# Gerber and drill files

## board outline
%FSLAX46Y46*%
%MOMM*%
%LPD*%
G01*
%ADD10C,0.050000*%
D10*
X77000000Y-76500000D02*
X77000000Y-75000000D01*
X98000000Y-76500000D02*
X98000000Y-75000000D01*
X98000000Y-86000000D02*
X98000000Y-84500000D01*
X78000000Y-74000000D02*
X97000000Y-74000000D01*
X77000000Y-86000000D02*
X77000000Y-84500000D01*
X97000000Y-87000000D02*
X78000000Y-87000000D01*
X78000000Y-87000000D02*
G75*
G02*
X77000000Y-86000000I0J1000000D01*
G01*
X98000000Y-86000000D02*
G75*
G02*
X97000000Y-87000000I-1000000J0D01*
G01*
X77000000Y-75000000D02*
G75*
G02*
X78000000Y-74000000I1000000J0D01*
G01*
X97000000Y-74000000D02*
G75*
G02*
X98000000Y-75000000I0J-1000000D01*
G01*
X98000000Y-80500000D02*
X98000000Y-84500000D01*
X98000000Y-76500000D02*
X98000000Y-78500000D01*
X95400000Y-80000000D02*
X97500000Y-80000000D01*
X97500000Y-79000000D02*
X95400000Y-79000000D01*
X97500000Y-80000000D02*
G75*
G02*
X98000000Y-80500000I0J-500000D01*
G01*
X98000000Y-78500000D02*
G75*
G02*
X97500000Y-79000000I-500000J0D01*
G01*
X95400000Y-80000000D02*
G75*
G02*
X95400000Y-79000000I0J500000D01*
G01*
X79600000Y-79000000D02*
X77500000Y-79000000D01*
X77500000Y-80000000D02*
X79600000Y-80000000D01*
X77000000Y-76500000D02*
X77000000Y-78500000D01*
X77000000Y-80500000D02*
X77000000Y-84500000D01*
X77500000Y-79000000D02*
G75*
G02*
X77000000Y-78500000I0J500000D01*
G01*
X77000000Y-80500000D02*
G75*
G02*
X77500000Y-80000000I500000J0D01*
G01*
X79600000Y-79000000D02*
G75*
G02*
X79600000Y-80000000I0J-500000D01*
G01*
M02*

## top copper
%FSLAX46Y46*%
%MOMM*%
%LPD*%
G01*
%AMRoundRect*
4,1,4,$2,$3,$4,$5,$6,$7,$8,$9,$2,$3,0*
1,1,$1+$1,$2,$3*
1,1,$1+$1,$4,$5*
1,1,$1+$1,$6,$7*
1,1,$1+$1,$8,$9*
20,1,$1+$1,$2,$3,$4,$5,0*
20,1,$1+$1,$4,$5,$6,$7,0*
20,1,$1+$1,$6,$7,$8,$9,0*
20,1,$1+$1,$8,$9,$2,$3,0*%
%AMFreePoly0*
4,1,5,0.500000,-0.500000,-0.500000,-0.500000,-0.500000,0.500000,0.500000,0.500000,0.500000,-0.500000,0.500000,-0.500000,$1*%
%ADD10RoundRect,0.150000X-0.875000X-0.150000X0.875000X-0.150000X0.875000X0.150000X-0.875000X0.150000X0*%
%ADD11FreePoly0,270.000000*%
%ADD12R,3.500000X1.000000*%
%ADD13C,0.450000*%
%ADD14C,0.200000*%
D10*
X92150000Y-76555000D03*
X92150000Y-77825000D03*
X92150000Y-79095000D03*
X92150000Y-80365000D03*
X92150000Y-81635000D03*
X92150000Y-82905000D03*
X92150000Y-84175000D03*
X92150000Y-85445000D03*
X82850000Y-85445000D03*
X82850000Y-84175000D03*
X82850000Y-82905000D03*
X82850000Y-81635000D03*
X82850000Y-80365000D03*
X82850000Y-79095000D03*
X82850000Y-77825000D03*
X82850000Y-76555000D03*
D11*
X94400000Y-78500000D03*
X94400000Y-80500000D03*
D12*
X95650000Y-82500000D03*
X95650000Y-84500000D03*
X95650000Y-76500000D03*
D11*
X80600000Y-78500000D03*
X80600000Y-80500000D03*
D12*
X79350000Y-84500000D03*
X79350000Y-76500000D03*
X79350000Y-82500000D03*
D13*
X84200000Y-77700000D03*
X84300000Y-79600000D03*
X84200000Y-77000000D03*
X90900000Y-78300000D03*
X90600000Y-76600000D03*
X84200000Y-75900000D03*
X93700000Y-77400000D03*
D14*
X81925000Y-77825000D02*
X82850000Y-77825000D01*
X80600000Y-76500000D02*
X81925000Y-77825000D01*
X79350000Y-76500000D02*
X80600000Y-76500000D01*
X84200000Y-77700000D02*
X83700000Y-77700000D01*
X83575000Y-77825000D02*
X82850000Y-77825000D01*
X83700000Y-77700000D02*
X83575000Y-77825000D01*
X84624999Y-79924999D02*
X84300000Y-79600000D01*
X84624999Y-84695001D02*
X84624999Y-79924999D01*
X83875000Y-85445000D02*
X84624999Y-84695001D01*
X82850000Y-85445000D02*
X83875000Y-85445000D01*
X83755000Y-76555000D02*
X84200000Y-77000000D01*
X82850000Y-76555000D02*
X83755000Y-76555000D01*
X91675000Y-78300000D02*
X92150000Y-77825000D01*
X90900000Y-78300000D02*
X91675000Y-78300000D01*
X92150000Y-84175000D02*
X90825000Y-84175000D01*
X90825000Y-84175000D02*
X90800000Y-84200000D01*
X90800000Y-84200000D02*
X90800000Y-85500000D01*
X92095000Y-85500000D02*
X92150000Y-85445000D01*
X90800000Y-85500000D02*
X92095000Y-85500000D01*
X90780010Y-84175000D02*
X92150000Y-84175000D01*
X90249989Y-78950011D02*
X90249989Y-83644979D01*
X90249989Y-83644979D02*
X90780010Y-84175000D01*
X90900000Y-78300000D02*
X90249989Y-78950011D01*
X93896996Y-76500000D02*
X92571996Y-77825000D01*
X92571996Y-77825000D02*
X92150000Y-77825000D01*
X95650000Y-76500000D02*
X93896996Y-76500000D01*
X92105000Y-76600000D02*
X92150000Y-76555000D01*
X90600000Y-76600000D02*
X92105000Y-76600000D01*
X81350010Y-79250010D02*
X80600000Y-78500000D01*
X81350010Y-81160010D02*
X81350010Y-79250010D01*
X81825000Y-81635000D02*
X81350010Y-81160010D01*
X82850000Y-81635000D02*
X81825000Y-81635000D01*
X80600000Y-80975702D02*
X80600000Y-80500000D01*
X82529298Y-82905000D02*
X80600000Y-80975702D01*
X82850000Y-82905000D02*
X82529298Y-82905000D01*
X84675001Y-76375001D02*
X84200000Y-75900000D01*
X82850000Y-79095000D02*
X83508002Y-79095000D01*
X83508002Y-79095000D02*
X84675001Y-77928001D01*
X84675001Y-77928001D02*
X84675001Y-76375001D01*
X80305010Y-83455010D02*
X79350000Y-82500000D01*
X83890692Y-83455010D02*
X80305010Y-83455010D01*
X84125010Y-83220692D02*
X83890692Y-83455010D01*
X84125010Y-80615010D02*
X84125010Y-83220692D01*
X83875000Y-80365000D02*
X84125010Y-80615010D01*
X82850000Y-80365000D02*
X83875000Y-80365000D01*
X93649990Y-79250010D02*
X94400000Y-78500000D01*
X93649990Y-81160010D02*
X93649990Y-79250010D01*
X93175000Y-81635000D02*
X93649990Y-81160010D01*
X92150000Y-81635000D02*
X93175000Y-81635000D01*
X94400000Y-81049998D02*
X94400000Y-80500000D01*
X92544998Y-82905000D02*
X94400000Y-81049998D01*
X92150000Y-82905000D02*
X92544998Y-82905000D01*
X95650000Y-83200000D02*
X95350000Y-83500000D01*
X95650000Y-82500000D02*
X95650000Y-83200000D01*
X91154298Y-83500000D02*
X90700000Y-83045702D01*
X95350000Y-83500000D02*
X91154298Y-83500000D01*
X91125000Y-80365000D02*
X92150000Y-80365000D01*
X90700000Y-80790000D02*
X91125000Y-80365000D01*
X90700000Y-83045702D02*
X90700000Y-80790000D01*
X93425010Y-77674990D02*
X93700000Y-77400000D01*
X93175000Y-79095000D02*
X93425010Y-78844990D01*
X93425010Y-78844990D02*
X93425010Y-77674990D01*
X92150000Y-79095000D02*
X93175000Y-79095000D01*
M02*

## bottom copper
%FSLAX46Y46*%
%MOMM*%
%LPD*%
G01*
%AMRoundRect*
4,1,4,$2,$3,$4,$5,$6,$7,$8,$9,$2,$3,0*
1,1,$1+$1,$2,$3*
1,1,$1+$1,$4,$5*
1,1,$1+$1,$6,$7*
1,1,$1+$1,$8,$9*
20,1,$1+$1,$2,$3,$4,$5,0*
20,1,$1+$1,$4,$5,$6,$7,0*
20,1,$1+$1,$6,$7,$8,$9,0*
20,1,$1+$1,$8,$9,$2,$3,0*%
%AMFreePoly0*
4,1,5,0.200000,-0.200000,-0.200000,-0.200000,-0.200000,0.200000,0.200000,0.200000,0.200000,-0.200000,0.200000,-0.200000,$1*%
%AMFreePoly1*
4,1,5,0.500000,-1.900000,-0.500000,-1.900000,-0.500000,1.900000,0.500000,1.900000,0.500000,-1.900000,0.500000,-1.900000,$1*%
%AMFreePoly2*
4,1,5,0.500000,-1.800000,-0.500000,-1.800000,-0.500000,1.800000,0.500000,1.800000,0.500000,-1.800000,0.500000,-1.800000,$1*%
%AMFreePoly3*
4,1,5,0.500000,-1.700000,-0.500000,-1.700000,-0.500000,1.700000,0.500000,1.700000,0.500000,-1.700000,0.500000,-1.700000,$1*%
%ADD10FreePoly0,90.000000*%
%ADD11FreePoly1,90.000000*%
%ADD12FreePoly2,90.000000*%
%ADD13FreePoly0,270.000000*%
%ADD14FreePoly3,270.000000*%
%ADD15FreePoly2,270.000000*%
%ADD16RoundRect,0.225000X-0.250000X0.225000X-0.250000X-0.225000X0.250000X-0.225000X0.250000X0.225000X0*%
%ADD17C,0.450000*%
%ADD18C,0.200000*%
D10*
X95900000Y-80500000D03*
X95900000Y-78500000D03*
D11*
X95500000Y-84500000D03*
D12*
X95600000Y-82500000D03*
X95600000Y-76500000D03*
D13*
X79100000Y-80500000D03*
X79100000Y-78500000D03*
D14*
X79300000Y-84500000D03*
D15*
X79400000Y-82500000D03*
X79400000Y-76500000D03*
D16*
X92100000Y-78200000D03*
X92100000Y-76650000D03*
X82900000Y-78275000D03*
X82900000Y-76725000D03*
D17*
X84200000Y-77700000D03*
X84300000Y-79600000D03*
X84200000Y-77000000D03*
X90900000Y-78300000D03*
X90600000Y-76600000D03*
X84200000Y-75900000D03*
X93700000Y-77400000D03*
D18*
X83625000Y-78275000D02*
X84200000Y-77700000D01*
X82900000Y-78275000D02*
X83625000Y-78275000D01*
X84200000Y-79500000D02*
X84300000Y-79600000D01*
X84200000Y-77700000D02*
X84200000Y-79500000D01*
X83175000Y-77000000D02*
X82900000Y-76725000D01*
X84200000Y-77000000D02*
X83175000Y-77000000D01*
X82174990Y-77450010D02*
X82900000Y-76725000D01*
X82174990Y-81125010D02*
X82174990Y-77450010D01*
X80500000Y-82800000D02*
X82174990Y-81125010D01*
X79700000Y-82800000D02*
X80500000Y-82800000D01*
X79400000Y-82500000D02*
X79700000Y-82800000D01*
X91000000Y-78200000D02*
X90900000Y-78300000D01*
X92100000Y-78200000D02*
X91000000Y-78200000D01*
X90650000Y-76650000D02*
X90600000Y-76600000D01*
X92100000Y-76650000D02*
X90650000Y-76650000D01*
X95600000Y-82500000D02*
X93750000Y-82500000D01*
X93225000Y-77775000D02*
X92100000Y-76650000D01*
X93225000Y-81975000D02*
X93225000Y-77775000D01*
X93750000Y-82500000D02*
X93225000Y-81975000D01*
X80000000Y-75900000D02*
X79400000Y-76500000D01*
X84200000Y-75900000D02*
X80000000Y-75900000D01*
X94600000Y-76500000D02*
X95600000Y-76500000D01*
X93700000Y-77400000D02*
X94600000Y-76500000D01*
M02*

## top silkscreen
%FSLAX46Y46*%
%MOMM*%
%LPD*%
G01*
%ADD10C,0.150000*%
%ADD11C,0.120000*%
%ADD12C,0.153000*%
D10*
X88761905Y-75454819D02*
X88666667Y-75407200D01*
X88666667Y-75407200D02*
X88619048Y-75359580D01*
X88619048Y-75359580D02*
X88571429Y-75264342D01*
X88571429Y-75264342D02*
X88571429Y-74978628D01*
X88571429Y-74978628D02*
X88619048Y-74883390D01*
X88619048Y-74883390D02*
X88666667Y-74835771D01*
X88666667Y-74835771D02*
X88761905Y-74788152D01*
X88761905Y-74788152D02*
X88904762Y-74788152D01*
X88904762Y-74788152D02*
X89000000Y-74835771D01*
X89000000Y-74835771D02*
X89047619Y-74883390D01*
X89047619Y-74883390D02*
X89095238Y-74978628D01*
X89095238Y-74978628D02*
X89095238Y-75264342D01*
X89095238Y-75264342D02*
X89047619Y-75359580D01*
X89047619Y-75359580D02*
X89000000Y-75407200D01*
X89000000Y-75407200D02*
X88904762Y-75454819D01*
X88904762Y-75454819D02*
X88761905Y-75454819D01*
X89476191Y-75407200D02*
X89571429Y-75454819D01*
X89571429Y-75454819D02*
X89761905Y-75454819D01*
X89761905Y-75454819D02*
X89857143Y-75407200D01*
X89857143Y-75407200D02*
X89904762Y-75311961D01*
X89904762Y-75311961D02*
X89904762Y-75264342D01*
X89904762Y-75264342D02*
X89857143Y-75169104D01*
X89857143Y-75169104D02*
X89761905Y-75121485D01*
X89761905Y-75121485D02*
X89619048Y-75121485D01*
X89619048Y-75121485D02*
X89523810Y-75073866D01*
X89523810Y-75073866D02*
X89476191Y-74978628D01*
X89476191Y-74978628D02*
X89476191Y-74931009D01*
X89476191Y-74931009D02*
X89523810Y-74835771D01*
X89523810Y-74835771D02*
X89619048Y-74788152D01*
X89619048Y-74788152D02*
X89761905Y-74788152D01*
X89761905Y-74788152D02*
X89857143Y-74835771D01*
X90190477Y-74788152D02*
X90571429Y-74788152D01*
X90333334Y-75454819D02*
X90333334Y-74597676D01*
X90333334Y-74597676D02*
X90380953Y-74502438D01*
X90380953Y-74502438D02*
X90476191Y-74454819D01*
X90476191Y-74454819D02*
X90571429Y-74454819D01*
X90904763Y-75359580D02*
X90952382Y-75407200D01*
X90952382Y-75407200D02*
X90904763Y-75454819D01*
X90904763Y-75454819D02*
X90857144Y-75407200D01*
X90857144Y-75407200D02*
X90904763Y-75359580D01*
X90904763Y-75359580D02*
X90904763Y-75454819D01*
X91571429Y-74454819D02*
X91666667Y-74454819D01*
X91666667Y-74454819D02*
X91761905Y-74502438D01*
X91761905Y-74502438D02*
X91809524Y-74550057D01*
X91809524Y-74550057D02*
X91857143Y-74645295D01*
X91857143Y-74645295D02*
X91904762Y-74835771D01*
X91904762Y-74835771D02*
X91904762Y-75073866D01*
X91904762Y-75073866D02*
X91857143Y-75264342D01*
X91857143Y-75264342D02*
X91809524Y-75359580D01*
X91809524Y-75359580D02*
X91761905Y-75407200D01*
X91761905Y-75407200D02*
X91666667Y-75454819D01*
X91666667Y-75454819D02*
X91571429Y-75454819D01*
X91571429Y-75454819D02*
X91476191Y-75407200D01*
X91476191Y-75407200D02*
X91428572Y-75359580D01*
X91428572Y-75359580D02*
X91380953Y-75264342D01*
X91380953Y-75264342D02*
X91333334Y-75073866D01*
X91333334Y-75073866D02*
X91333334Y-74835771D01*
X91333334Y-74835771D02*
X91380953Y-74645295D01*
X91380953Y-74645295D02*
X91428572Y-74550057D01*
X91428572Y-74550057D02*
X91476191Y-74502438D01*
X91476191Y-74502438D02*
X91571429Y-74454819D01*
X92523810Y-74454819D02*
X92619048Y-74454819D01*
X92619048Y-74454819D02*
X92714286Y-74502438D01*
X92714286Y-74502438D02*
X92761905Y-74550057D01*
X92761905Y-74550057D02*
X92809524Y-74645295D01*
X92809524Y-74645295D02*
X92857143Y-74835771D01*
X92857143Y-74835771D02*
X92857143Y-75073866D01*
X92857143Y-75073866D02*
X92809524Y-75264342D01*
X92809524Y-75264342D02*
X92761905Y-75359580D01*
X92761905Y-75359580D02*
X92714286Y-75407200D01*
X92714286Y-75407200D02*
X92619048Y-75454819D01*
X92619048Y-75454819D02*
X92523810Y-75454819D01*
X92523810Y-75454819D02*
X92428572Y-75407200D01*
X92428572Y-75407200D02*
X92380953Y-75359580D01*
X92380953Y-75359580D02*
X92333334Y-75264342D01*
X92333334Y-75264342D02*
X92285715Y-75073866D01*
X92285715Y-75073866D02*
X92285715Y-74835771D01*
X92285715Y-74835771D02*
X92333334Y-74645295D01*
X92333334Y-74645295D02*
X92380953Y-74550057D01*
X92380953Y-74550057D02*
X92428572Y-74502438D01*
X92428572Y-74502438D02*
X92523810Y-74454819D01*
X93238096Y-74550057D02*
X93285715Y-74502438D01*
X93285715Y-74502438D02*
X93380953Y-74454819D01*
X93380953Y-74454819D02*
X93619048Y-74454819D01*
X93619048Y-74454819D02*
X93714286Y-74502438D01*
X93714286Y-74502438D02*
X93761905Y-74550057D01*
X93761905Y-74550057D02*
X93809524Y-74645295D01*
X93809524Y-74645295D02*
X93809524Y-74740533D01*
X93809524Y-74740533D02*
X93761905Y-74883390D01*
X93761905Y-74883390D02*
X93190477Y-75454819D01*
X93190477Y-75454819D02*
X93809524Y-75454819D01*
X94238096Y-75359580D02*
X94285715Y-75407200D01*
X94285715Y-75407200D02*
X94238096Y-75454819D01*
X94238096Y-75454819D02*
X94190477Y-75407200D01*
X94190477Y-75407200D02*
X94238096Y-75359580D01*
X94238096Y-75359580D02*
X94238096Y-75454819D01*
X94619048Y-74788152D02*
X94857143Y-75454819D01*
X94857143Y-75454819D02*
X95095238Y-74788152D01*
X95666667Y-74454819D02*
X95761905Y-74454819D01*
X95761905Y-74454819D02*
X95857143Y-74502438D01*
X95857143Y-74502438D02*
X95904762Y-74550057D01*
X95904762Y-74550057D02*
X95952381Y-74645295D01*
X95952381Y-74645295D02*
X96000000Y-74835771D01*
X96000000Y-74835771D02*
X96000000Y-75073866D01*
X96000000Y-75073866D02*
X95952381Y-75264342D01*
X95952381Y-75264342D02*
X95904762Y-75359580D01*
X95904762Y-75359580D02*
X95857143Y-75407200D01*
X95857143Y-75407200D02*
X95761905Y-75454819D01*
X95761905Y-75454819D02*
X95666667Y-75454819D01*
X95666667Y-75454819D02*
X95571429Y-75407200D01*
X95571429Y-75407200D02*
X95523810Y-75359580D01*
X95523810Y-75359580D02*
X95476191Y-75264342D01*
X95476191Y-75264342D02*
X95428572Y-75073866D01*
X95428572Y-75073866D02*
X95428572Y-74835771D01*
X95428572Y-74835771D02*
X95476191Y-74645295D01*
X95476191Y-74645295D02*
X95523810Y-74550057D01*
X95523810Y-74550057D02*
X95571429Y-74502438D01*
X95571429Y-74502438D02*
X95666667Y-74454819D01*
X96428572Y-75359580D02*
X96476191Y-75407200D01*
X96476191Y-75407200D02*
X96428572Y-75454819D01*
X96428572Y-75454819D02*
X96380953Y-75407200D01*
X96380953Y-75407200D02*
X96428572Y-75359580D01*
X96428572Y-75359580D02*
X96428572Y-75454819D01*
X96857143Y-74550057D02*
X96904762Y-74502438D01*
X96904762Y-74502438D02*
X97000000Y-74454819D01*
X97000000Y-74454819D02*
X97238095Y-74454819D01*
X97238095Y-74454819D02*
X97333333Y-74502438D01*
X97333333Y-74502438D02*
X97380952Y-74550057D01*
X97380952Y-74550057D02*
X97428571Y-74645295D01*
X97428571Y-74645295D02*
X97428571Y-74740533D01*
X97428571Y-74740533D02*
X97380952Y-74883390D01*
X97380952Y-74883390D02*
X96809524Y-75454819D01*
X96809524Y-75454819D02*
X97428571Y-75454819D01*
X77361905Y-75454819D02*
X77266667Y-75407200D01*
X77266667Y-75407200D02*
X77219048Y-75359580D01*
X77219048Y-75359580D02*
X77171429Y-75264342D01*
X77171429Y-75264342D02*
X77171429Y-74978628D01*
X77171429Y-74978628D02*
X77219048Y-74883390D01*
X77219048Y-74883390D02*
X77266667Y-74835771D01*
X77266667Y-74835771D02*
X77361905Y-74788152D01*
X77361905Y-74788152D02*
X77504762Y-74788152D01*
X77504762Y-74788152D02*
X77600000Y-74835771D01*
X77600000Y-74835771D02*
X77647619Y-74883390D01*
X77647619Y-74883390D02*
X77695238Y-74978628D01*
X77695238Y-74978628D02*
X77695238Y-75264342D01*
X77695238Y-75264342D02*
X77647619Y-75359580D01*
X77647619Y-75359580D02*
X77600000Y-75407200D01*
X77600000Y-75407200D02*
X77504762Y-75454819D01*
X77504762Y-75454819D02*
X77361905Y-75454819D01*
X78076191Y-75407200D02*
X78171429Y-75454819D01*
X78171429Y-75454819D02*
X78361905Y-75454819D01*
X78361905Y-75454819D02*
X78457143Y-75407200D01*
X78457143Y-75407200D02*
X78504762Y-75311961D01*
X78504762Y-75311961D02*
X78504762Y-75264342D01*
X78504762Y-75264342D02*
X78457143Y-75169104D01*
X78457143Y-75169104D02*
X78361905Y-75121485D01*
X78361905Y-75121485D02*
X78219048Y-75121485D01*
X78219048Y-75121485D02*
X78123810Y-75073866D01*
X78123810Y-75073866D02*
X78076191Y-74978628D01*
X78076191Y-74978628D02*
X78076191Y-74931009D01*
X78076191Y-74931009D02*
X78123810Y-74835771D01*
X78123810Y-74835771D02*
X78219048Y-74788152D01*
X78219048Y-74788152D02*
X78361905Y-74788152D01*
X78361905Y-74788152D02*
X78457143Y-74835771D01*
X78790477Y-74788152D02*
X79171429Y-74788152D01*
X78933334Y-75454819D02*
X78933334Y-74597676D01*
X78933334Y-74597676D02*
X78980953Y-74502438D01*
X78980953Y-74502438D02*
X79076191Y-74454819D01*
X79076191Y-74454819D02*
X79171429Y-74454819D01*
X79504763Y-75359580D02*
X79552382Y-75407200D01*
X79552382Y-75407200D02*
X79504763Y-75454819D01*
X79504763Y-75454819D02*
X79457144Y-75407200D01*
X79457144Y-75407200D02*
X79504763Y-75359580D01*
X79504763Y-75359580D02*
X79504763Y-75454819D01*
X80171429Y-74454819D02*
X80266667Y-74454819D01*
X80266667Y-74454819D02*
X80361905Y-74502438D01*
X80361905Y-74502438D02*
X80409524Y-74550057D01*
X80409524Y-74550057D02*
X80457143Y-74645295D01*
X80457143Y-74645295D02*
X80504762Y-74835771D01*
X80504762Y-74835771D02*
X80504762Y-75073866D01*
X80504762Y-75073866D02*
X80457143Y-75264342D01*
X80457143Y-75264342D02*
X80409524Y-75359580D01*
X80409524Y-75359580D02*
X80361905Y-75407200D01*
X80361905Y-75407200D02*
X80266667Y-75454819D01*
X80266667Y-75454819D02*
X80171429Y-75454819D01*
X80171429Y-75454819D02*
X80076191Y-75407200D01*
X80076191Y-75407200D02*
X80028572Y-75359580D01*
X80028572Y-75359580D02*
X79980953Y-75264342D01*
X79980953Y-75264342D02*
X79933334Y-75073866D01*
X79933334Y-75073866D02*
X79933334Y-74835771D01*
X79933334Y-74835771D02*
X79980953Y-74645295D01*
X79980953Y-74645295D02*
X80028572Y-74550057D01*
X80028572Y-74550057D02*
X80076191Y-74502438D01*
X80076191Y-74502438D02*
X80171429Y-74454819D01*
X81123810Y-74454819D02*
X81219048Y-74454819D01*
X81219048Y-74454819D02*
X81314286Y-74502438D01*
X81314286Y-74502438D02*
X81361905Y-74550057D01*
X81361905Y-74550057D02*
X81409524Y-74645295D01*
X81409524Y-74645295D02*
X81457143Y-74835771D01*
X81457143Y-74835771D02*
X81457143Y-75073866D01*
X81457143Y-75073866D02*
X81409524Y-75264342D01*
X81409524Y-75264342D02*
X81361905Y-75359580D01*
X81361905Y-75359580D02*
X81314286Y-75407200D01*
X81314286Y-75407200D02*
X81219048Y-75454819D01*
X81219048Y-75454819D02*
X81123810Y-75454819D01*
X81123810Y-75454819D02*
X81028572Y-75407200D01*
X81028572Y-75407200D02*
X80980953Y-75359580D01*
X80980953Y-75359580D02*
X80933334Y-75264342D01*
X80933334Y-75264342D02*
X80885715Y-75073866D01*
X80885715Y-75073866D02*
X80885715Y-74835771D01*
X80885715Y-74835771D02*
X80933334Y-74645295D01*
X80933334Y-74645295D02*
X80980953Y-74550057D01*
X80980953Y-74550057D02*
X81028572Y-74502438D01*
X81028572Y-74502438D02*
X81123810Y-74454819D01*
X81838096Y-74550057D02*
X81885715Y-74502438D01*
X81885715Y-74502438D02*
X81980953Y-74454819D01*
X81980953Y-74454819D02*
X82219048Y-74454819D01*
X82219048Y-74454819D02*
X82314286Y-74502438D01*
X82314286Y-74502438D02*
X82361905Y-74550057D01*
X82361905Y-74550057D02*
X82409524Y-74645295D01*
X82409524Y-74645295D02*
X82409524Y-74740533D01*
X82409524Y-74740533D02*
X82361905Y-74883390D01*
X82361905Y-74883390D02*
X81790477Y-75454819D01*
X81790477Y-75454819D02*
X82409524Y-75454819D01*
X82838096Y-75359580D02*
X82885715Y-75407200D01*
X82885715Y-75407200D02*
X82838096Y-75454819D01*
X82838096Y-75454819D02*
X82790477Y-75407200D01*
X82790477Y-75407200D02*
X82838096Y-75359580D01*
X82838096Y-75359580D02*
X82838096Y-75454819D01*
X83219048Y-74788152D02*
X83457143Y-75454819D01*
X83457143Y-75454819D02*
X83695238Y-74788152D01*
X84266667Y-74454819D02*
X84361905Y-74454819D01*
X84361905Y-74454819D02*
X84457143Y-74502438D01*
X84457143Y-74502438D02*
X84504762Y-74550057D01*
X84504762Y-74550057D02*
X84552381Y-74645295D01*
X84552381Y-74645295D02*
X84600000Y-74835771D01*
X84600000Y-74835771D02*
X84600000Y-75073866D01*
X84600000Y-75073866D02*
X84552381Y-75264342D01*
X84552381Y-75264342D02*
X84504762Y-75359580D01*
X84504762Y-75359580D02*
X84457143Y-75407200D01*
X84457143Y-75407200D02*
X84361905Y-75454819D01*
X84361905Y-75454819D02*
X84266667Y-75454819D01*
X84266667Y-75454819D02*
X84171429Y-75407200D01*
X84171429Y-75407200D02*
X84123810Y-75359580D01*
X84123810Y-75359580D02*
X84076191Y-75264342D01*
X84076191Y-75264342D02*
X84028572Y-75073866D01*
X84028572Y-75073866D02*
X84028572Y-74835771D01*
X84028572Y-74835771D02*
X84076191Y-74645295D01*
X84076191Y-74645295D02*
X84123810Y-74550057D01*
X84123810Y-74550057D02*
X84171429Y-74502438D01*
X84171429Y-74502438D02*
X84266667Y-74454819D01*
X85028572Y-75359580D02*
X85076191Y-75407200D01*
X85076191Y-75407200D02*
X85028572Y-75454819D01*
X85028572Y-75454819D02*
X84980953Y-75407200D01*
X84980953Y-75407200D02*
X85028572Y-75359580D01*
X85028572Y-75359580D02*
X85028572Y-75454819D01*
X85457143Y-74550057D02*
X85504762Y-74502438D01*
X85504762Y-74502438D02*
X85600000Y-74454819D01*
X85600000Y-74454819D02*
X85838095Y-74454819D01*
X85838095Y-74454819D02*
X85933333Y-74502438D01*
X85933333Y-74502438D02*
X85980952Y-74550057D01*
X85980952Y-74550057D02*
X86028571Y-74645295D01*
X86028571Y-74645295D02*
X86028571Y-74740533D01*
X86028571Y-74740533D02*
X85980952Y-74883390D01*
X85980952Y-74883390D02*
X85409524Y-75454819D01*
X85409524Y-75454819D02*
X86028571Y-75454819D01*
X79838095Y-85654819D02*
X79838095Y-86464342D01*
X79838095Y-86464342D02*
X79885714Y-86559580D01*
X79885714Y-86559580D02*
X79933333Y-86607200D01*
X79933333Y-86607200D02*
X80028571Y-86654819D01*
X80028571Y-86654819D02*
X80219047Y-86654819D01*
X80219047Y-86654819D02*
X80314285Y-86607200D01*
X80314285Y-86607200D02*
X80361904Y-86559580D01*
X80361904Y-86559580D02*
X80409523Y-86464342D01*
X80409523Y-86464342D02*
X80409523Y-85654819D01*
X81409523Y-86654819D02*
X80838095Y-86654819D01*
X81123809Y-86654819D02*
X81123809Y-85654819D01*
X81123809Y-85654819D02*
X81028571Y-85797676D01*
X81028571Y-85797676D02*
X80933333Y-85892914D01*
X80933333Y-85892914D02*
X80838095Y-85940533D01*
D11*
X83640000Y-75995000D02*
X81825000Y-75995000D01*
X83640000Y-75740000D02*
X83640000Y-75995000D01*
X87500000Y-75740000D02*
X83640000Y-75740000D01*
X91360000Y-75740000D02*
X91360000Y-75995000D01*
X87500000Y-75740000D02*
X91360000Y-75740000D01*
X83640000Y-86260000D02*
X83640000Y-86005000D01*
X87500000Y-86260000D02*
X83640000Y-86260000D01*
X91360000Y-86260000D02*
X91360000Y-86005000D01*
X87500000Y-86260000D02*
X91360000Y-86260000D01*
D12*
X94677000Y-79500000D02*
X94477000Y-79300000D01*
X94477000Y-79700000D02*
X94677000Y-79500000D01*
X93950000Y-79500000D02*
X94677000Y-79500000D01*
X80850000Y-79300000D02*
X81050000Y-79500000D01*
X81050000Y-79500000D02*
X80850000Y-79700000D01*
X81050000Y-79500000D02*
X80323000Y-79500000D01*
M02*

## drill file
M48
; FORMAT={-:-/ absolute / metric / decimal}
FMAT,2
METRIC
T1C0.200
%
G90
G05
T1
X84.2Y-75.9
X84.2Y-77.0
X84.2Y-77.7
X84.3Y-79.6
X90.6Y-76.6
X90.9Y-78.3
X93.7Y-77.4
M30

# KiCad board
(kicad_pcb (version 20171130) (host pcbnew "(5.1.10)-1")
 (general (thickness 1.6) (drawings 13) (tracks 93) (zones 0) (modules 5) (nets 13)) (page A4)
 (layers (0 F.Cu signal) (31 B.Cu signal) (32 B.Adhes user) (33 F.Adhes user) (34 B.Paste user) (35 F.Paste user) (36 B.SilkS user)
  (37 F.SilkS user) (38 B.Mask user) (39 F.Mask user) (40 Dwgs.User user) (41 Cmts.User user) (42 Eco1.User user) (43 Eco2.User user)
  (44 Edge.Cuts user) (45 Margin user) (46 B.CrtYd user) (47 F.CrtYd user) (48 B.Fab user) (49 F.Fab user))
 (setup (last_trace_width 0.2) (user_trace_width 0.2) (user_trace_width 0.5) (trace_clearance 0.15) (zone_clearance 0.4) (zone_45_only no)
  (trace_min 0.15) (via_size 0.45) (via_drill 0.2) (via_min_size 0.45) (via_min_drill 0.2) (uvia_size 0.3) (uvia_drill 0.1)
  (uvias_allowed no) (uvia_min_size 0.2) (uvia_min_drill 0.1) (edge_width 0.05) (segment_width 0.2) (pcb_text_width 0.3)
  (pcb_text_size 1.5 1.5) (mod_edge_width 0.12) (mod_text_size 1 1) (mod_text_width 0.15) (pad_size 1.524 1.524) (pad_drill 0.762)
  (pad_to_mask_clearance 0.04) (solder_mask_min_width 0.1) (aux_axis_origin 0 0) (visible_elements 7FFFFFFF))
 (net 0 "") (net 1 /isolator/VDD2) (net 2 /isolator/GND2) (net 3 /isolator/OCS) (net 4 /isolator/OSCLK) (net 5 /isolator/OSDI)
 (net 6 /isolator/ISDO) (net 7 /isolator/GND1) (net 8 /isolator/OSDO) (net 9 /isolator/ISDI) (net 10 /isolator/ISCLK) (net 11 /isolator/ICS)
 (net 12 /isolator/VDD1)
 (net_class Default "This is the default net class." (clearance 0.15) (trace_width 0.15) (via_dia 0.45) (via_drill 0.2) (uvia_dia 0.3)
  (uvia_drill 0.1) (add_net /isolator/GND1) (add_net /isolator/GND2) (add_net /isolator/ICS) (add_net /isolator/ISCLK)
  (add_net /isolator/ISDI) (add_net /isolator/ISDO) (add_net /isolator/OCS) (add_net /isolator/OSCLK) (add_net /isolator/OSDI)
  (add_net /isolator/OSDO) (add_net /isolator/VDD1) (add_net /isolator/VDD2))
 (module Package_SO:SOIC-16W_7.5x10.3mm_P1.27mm (layer F.Cu) (at 87.5 81)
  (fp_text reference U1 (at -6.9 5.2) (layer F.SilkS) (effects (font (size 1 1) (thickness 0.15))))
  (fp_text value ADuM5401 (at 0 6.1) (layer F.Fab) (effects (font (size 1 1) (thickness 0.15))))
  (fp_line (start -3.86 -5.005) (end -5.675 -5.005) (layer F.SilkS) (width 0.12))
  (fp_line (start -3.86 -5.26) (end -3.86 -5.005) (layer F.SilkS) (width 0.12))
  (fp_line (start 0 -5.26) (end -3.86 -5.26) (layer F.SilkS) (width 0.12))
  (fp_line (start 3.86 -5.26) (end 3.86 -5.005) (layer F.SilkS) (width 0.12))
  (fp_line (start 0 -5.26) (end 3.86 -5.26) (layer F.SilkS) (width 0.12))
  (fp_line (start -3.86 5.26) (end -3.86 5.005) (layer F.SilkS) (width 0.12))
  (fp_line (start 0 5.26) (end -3.86 5.26) (layer F.SilkS) (width 0.12))
  (fp_line (start 3.86 5.26) (end 3.86 5.005) (layer F.SilkS) (width 0.12))
  (fp_line (start 0 5.26) (end 3.86 5.26) (layer F.SilkS) (width 0.12))
  (pad 16 smd roundrect (at 4.65 -4.445) (size 2.05 0.6) (layers F.Cu F.Paste F.Mask) (roundrect_rratio 0.25) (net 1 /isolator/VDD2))
  (pad 15 smd roundrect (at 4.65 -3.175) (size 2.05 0.6) (layers F.Cu F.Paste F.Mask) (roundrect_rratio 0.25) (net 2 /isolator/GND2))
  (pad 14 smd roundrect (at 4.65 -1.905) (size 2.05 0.6) (layers F.Cu F.Paste F.Mask) (roundrect_rratio 0.25) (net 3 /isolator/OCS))
  (pad 13 smd roundrect (at 4.65 -0.635) (size 2.05 0.6) (layers F.Cu F.Paste F.Mask) (roundrect_rratio 0.25) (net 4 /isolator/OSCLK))
  (pad 12 smd roundrect (at 4.65 0.635) (size 2.05 0.6) (layers F.Cu F.Paste F.Mask) (roundrect_rratio 0.25) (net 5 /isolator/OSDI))
  (pad 11 smd roundrect (at 4.65 1.905) (size 2.05 0.6) (layers F.Cu F.Paste F.Mask) (roundrect_rratio 0.25) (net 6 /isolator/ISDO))
  (pad 10 smd roundrect (at 4.65 3.175) (size 2.05 0.6) (layers F.Cu F.Paste F.Mask) (roundrect_rratio 0.25) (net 2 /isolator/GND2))
  (pad 9 smd roundrect (at 4.65 4.445) (size 2.05 0.6) (layers F.Cu F.Paste F.Mask) (roundrect_rratio 0.25) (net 2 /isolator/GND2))
  (pad 8 smd roundrect (at -4.65 4.445) (size 2.05 0.6) (layers F.Cu F.Paste F.Mask) (roundrect_rratio 0.25) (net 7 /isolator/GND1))
  (pad 7 smd roundrect (at -4.65 3.175) (size 2.05 0.6) (layers F.Cu F.Paste F.Mask) (roundrect_rratio 0.25))
  (pad 6 smd roundrect (at -4.65 1.905) (size 2.05 0.6) (layers F.Cu F.Paste F.Mask) (roundrect_rratio 0.25) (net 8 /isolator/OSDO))
  (pad 5 smd roundrect (at -4.65 0.635) (size 2.05 0.6) (layers F.Cu F.Paste F.Mask) (roundrect_rratio 0.25) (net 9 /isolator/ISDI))
  (pad 4 smd roundrect (at -4.65 -0.635) (size 2.05 0.6) (layers F.Cu F.Paste F.Mask) (roundrect_rratio 0.25) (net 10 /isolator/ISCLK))
  (pad 3 smd roundrect (at -4.65 -1.905) (size 2.05 0.6) (layers F.Cu F.Paste F.Mask) (roundrect_rratio 0.25) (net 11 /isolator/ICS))
  (pad 2 smd roundrect (at -4.65 -3.175) (size 2.05 0.6) (layers F.Cu F.Paste F.Mask) (roundrect_rratio 0.25) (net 7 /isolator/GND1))
  (pad 1 smd roundrect (at -4.65 -4.445) (size 2.05 0.6) (layers F.Cu F.Paste F.Mask) (roundrect_rratio 0.25) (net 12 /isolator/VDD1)))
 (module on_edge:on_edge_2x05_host (layer F.Cu) (at 98 80.5 270)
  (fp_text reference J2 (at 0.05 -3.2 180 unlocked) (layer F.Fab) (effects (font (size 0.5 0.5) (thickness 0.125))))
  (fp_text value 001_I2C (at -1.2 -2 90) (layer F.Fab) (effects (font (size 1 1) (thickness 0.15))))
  (fp_line (start 0 0) (end 4 0) (layer Edge.Cuts) (width 0.05))
  (fp_line (start -4 0) (end -2 0) (layer Edge.Cuts) (width 0.05))
  (fp_line (start -0.5 2.6) (end -0.5 0.5) (layer Edge.Cuts) (width 0.05))
  (fp_line (start -1.5 0.5) (end -1.5 2.6) (layer Edge.Cuts) (width 0.05))
  (fp_line (start -1 3.323) (end -1.2 3.523) (layer F.SilkS) (width 0.153))
  (fp_line (start -0.8 3.523) (end -1 3.323) (layer F.SilkS) (width 0.153))
  (fp_line (start -1 4.05) (end -1 3.323) (layer F.SilkS) (width 0.153))
  (fp_arc (start 0 0.5) (end 0 0) (angle -90) (layer Edge.Cuts) (width 0.05))
  (fp_arc (start -2 0.5) (end -1.5 0.5) (angle -90) (layer Edge.Cuts) (width 0.05))
  (fp_arc (start -1 2.6) (end -1.5 2.6) (angle -180) (layer Edge.Cuts) (width 0.05))
  (pad 2 smd custom (at -2 3.6 270) (size 1 1) (layers F.Cu F.Mask) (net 5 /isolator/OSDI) (zone_connect 0)
   (options (clearance outline) (anchor rect)) (primitives))
  (pad 3 smd custom (at 0 3.6 270) (size 1 1) (layers F.Cu F.Mask) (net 6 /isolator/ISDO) (zone_connect 0)
   (options (clearance outline) (anchor rect)) (primitives))
  (pad 8 smd custom (at 0 2.1 90) (size 0.4 0.4) (layers B.Cu B.Mask) (zone_connect 0) (options (clearance outline) (anchor rect))
   (primitives))
  (pad 7 smd custom (at -2 2.1 90) (size 0.4 0.4) (layers B.Cu B.Mask) (zone_connect 0) (options (clearance outline) (anchor rect))
   (primitives))
  (pad 4 smd rect (at 2 2.35 270) (size 1 3.5) (layers F.Cu F.Mask) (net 4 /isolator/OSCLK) (zone_connect 0))
  (pad 10 smd custom (at 4 2.5 90) (size 1 3.8) (layers B.Cu B.Mask) (zone_connect 0) (options (clearance outline) (anchor rect))
   (primitives))
  (pad 9 smd custom (at 2 2.4 90) (size 1 3.6) (layers B.Cu B.Mask) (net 1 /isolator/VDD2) (zone_connect 0)
   (options (clearance outline) (anchor rect)) (primitives))
  (pad 6 smd custom (at -4 2.4 90) (size 1 3.6) (layers B.Cu B.Mask) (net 3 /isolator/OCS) (zone_connect 0)
   (options (clearance outline) (anchor rect)) (primitives))
  (pad 5 smd rect (at 4 2.35 270) (size 1 3.5) (layers F.Cu F.Mask) (zone_connect 0))
  (pad 1 smd rect (at -4 2.35 270) (size 1 3.5) (layers F.Cu F.Mask) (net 2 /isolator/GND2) (zone_connect 0)))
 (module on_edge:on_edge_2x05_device (layer F.Cu) (at 77 80.5 270)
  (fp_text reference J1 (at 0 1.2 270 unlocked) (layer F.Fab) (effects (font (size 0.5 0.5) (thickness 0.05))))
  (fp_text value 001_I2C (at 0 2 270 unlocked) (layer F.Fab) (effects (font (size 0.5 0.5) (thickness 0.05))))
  (fp_line (start -1.5 -2.6) (end -1.5 -0.5) (layer Edge.Cuts) (width 0.05))
  (fp_line (start -0.5 -0.5) (end -0.5 -2.6) (layer Edge.Cuts) (width 0.05))
  (fp_line (start -1.2 -3.85) (end -1 -4.05) (layer F.SilkS) (width 0.153))
  (fp_line (start -1 -4.05) (end -0.8 -3.85) (layer F.SilkS) (width 0.153))
  (fp_line (start -1 -4.05) (end -1 -3.323) (layer F.SilkS) (width 0.153))
  (fp_line (start -4 0) (end -2 0) (layer Edge.Cuts) (width 0.05))
  (fp_line (start 0 0) (end 4 0) (layer Edge.Cuts) (width 0.05))
  (fp_arc (start -2 -0.5) (end -2 0) (angle -90) (layer Edge.Cuts) (width 0.05))
  (fp_arc (start 0 -0.5) (end -0.5 -0.5) (angle -90) (layer Edge.Cuts) (width 0.05))
  (fp_arc (start -1 -2.6) (end -0.5 -2.6) (angle -180) (layer Edge.Cuts) (width 0.05))
  (pad 2 smd custom (at -2 -3.6 270) (size 1 1) (layers F.Cu F.Mask) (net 9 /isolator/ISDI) (zone_connect 0)
   (options (clearance outline) (anchor rect)) (primitives))
  (pad 3 smd custom (at 0 -3.6 270) (size 1 1) (layers F.Cu F.Mask) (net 8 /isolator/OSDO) (zone_connect 0)
   (options (clearance outline) (anchor rect)) (primitives))
  (pad 8 smd custom (at 0 -2.1 270) (size 0.4 0.4) (layers B.Cu B.Mask) (zone_connect 0) (options (clearance outline) (anchor rect))
   (primitives))
  (pad 7 smd custom (at -2 -2.1 270) (size 0.4 0.4) (layers B.Cu B.Mask) (zone_connect 0) (options (clearance outline) (anchor rect))
   (primitives))
  (pad 10 smd custom (at 4 -2.3 270) (size 1 3.4) (layers B.Cu B.Mask) (zone_connect 0) (options (clearance outline) (anchor rect))
   (primitives))
  (pad 9 smd custom (at 2 -2.4 270) (size 1 3.6) (layers B.Cu B.Mask) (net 12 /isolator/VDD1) (zone_connect 0)
   (options (clearance outline) (anchor rect)) (primitives))
  (pad 6 smd custom (at -4 -2.4 270) (size 1 3.6) (layers B.Cu B.Mask) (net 11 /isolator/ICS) (zone_connect 0)
   (options (clearance outline) (anchor rect)) (primitives))
  (pad 5 smd rect (at 4 -2.35 90) (size 1 3.5) (layers F.Cu F.Mask) (zone_connect 0))
  (pad 1 smd rect (at -4 -2.35 90) (size 1 3.5) (layers F.Cu F.Mask) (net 7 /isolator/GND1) (zone_connect 0))
  (pad 4 smd rect (at 2 -2.35 90) (size 1 3.5) (layers F.Cu F.Mask) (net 10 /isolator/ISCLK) (zone_connect 0)))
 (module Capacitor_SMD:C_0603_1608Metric (layer B.Cu) (at 92.1 77.425 270)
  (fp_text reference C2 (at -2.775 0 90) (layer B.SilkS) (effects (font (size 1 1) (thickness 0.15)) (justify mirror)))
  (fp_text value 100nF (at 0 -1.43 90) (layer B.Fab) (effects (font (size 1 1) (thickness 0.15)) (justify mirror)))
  (pad 2 smd roundrect (at 0.775 0 270) (size 0.9 0.95) (layers B.Cu B.Paste B.Mask) (roundrect_rratio 0.25) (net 2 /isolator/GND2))
  (pad 1 smd roundrect (at -0.775 0 270) (size 0.9 0.95) (layers B.Cu B.Paste B.Mask) (roundrect_rratio 0.25) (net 1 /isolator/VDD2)))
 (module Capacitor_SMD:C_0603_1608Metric (layer B.Cu) (at 82.9 77.5 270)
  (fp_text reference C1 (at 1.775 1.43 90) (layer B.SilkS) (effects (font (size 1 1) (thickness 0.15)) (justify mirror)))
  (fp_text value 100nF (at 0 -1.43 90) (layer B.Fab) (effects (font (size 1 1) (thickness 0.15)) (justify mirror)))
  (pad 2 smd roundrect (at 0.775 0 270) (size 0.9 0.95) (layers B.Cu B.Paste B.Mask) (roundrect_rratio 0.25) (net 7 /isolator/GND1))
  (pad 1 smd roundrect (at -0.775 0 270) (size 0.9 0.95) (layers B.Cu B.Paste B.Mask) (roundrect_rratio 0.25) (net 12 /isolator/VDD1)))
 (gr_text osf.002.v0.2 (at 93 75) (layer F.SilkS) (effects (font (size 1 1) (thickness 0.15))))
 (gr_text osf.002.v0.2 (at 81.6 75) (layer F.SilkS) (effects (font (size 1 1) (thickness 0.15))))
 (gr_line (start 77 76.5) (end 77 75) (layer Edge.Cuts) (width 0.05))
 (gr_line (start 98 76.5) (end 98 75) (layer Edge.Cuts) (width 0.05))
 (gr_line (start 98 86) (end 98 84.5) (layer Edge.Cuts) (width 0.05))
 (gr_line (start 78 74) (end 97 74) (layer Edge.Cuts) (width 0.05))
 (gr_line (start 77 86) (end 77 84.5) (layer Edge.Cuts) (width 0.05))
 (gr_line (start 97 87) (end 78 87) (layer Edge.Cuts) (width 0.05))
 (gr_arc (start 78 86) (end 77 86) (angle -90) (layer Edge.Cuts) (width 0.05))
 (gr_arc (start 97 86) (end 97 87) (angle -90) (layer Edge.Cuts) (width 0.05))
 (gr_arc (start 78 75) (end 78 74) (angle -90) (layer Edge.Cuts) (width 0.05))
 (gr_arc (start 97 75) (end 98 75) (angle -90) (layer Edge.Cuts) (width 0.05))
 (segment (start 81.925 77.825) (end 82.85 77.825) (width 0.2) (layer F.Cu) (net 7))
 (segment (start 80.6 76.5) (end 81.925 77.825) (width 0.2) (layer F.Cu) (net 7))
 (segment (start 79.35 76.5) (end 80.6 76.5) (width 0.2) (layer F.Cu) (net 7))
 (via (at 84.2 77.7) (size 0.45) (drill 0.2) (layers F.Cu B.Cu) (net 7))
 (segment (start 84.2 77.7) (end 83.7 77.7) (width 0.2) (layer F.Cu) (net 7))
 (segment (start 83.575 77.825) (end 82.85 77.825) (width 0.2) (layer F.Cu) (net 7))
 (segment (start 83.7 77.7) (end 83.575 77.825) (width 0.2) (layer F.Cu) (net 7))
 (segment (start 83.625 78.275) (end 84.2 77.7) (width 0.2) (layer B.Cu) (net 7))
 (segment (start 82.9 78.275) (end 83.625 78.275) (width 0.2) (layer B.Cu) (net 7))
 (segment (start 84.624999 79.924999) (end 84.3 79.6) (width 0.2) (layer F.Cu) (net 7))
 (segment (start 84.624999 84.695001) (end 84.624999 79.924999) (width 0.2) (layer F.Cu) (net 7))
 (segment (start 83.875 85.445) (end 84.624999 84.695001) (width 0.2) (layer F.Cu) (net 7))
 (segment (start 82.85 85.445) (end 83.875 85.445) (width 0.2) (layer F.Cu) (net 7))
 (segment (start 84.2 79.5) (end 84.3 79.6) (width 0.2) (layer B.Cu) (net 7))
 (segment (start 84.2 77.7) (end 84.2 79.5) (width 0.2) (layer B.Cu) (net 7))
 (via (at 84.3 79.6) (size 0.45) (drill 0.2) (layers F.Cu B.Cu) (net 7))
 (via (at 84.2 77) (size 0.45) (drill 0.2) (layers F.Cu B.Cu) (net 12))
 (segment (start 83.755 76.555) (end 84.2 77) (width 0.2) (layer F.Cu) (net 12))
 (segment (start 82.85 76.555) (end 83.755 76.555) (width 0.2) (layer F.Cu) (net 12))
 (segment (start 83.175 77) (end 82.9 76.725) (width 0.2) (layer B.Cu) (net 12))
 (segment (start 84.2 77) (end 83.175 77) (width 0.2) (layer B.Cu) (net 12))
 (segment (start 82.17499 77.45001) (end 82.9 76.725) (width 0.2) (layer B.Cu) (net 12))
 (segment (start 82.17499 81.12501) (end 82.17499 77.45001) (width 0.2) (layer B.Cu) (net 12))
 (segment (start 80.5 82.8) (end 82.17499 81.12501) (width 0.2) (layer B.Cu) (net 12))
 (segment (start 79.7 82.8) (end 80.5 82.8) (width 0.2) (layer B.Cu) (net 12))
 (segment (start 79.4 82.5) (end 79.7 82.8) (width 0.2) (layer B.Cu) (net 12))
 (segment (start 91 78.2) (end 90.9 78.3) (width 0.2) (layer B.Cu) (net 2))
 (segment (start 92.1 78.2) (end 91 78.2) (width 0.2) (layer B.Cu) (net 2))
 (via (at 90.9 78.3) (size 0.45) (drill 0.2) (layers F.Cu B.Cu) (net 2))
 (segment (start 91.675 78.3) (end 92.15 77.825) (width 0.2) (layer F.Cu) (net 2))
 (segment (start 90.9 78.3) (end 91.675 78.3) (width 0.2) (layer F.Cu) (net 2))
 (segment (start 92.15 84.175) (end 90.825 84.175) (width 0.2) (layer F.Cu) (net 2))
 (segment (start 90.825 84.175) (end 90.8 84.2) (width 0.2) (layer F.Cu) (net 2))
 (segment (start 90.8 84.2) (end 90.8 85.5) (width 0.2) (layer F.Cu) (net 2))
 (segment (start 92.095 85.5) (end 92.15 85.445) (width 0.2) (layer F.Cu) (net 2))
 (segment (start 90.8 85.5) (end 92.095 85.5) (width 0.2) (layer F.Cu) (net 2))
 (segment (start 90.78001 84.175) (end 92.15 84.175) (width 0.2) (layer F.Cu) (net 2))
 (segment (start 90.249989 78.950011) (end 90.249989 83.644979) (width 0.2) (layer F.Cu) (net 2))
 (segment (start 90.249989 83.644979) (end 90.78001 84.175) (width 0.2) (layer F.Cu) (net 2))
 (segment (start 90.9 78.3) (end 90.249989 78.950011) (width 0.2) (layer F.Cu) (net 2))
 (segment (start 93.896996 76.5) (end 92.571996 77.825) (width 0.2) (layer F.Cu) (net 2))
 (segment (start 92.571996 77.825) (end 92.15 77.825) (width 0.2) (layer F.Cu) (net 2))
 (segment (start 95.65 76.5) (end 93.896996 76.5) (width 0.2) (layer F.Cu) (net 2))
 (segment (start 90.65 76.65) (end 90.6 76.6) (width 0.2) (layer B.Cu) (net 1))
 (via (at 90.6 76.6) (size 0.45) (drill 0.2) (layers F.Cu B.Cu) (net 1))
 (segment (start 92.1 76.65) (end 90.65 76.65) (width 0.2) (layer B.Cu) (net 1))
 (segment (start 92.105 76.6) (end 92.15 76.555) (width 0.2) (layer F.Cu) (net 1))
 (segment (start 90.6 76.6) (end 92.105 76.6) (width 0.2) (layer F.Cu) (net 1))
 (segment (start 95.6 82.5) (end 93.75 82.5) (width 0.2) (layer B.Cu) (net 1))
 (segment (start 93.225 77.775) (end 92.1 76.65) (width 0.2) (layer B.Cu) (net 1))
 (segment (start 93.225 81.975) (end 93.225 77.775) (width 0.2) (layer B.Cu) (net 1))
 (segment (start 93.75 82.5) (end 93.225 81.975) (width 0.2) (layer B.Cu) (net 1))
 (segment (start 81.35001 79.25001) (end 80.6 78.5) (width 0.2) (layer F.Cu) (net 9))
 (segment (start 81.35001 81.16001) (end 81.35001 79.25001) (width 0.2) (layer F.Cu) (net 9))
 (segment (start 81.825 81.635) (end 81.35001 81.16001) (width 0.2) (layer F.Cu) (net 9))
 (segment (start 82.85 81.635) (end 81.825 81.635) (width 0.2) (layer F.Cu) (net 9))
 (segment (start 80.6 80.975702) (end 80.6 80.5) (width 0.2) (layer F.Cu) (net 8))
 (segment (start 82.529298 82.905) (end 80.6 80.975702) (width 0.2) (layer F.Cu) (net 8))
 (segment (start 82.85 82.905) (end 82.529298 82.905) (width 0.2) (layer F.Cu) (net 8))
 (via (at 84.2 75.9) (size 0.45) (drill 0.2) (layers F.Cu B.Cu) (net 11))
 (segment (start 80 75.9) (end 79.4 76.5) (width 0.2) (layer B.Cu) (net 11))
 (segment (start 84.2 75.9) (end 80 75.9) (width 0.2) (layer B.Cu) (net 11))
 (segment (start 84.675001 76.375001) (end 84.2 75.9) (width 0.2) (layer F.Cu) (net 11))
 (segment (start 82.85 79.095) (end 83.508002 79.095) (width 0.2) (layer F.Cu) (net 11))
 (segment (start 83.508002 79.095) (end 84.675001 77.928001) (width 0.2) (layer F.Cu) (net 11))
 (segment (start 84.675001 77.928001) (end 84.675001 76.375001) (width 0.2) (layer F.Cu) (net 11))
 (segment (start 80.30501 83.45501) (end 79.35 82.5) (width 0.2) (layer F.Cu) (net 10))
 (segment (start 83.890692 83.45501) (end 80.30501 83.45501) (width 0.2) (layer F.Cu) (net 10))
 (segment (start 84.12501 83.220692) (end 83.890692 83.45501) (width 0.2) (layer F.Cu) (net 10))
 (segment (start 84.12501 80.61501) (end 84.12501 83.220692) (width 0.2) (layer F.Cu) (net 10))
 (segment (start 83.875 80.365) (end 84.12501 80.61501) (width 0.2) (layer F.Cu) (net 10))
 (segment (start 82.85 80.365) (end 83.875 80.365) (width 0.2) (layer F.Cu) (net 10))
 (segment (start 93.64999 79.25001) (end 94.4 78.5) (width 0.2) (layer F.Cu) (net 5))
 (segment (start 93.64999 81.16001) (end 93.64999 79.25001) (width 0.2) (layer F.Cu) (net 5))
 (segment (start 93.175 81.635) (end 93.64999 81.16001) (width 0.2) (layer F.Cu) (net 5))
 (segment (start 92.15 81.635) (end 93.175 81.635) (width 0.2) (layer F.Cu) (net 5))
 (segment (start 94.4 81.049998) (end 94.4 80.5) (width 0.2) (layer F.Cu) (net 6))
 (segment (start 92.544998 82.905) (end 94.4 81.049998) (width 0.2) (layer F.Cu) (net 6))
 (segment (start 92.15 82.905) (end 92.544998 82.905) (width 0.2) (layer F.Cu) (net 6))
 (segment (start 95.65 83.2) (end 95.35 83.5) (width 0.2) (layer F.Cu) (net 4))
 (segment (start 95.65 82.5) (end 95.65 83.2) (width 0.2) (layer F.Cu) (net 4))
 (segment (start 91.154298 83.5) (end 90.7 83.045702) (width 0.2) (layer F.Cu) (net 4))
 (segment (start 95.35 83.5) (end 91.154298 83.5) (width 0.2) (layer F.Cu) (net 4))
 (segment (start 91.125 80.365) (end 92.15 80.365) (width 0.2) (layer F.Cu) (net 4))
 (segment (start 90.7 80.79) (end 91.125 80.365) (width 0.2) (layer F.Cu) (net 4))
 (segment (start 90.7 83.045702) (end 90.7 80.79) (width 0.2) (layer F.Cu) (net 4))
 (via (at 93.7 77.4) (size 0.45) (drill 0.2) (layers F.Cu B.Cu) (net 3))
 (segment (start 93.42501 77.67499) (end 93.7 77.4) (width 0.2) (layer F.Cu) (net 3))
 (segment (start 93.175 79.095) (end 93.42501 78.84499) (width 0.2) (layer F.Cu) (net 3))
 (segment (start 93.42501 78.84499) (end 93.42501 77.67499) (width 0.2) (layer F.Cu) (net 3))
 (segment (start 92.15 79.095) (end 93.175 79.095) (width 0.2) (layer F.Cu) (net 3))
 (segment (start 94.6 76.5) (end 95.6 76.5) (width 0.2) (layer B.Cu) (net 3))
 (segment (start 93.7 77.4) (end 94.6 76.5) (width 0.2) (layer B.Cu) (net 3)))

